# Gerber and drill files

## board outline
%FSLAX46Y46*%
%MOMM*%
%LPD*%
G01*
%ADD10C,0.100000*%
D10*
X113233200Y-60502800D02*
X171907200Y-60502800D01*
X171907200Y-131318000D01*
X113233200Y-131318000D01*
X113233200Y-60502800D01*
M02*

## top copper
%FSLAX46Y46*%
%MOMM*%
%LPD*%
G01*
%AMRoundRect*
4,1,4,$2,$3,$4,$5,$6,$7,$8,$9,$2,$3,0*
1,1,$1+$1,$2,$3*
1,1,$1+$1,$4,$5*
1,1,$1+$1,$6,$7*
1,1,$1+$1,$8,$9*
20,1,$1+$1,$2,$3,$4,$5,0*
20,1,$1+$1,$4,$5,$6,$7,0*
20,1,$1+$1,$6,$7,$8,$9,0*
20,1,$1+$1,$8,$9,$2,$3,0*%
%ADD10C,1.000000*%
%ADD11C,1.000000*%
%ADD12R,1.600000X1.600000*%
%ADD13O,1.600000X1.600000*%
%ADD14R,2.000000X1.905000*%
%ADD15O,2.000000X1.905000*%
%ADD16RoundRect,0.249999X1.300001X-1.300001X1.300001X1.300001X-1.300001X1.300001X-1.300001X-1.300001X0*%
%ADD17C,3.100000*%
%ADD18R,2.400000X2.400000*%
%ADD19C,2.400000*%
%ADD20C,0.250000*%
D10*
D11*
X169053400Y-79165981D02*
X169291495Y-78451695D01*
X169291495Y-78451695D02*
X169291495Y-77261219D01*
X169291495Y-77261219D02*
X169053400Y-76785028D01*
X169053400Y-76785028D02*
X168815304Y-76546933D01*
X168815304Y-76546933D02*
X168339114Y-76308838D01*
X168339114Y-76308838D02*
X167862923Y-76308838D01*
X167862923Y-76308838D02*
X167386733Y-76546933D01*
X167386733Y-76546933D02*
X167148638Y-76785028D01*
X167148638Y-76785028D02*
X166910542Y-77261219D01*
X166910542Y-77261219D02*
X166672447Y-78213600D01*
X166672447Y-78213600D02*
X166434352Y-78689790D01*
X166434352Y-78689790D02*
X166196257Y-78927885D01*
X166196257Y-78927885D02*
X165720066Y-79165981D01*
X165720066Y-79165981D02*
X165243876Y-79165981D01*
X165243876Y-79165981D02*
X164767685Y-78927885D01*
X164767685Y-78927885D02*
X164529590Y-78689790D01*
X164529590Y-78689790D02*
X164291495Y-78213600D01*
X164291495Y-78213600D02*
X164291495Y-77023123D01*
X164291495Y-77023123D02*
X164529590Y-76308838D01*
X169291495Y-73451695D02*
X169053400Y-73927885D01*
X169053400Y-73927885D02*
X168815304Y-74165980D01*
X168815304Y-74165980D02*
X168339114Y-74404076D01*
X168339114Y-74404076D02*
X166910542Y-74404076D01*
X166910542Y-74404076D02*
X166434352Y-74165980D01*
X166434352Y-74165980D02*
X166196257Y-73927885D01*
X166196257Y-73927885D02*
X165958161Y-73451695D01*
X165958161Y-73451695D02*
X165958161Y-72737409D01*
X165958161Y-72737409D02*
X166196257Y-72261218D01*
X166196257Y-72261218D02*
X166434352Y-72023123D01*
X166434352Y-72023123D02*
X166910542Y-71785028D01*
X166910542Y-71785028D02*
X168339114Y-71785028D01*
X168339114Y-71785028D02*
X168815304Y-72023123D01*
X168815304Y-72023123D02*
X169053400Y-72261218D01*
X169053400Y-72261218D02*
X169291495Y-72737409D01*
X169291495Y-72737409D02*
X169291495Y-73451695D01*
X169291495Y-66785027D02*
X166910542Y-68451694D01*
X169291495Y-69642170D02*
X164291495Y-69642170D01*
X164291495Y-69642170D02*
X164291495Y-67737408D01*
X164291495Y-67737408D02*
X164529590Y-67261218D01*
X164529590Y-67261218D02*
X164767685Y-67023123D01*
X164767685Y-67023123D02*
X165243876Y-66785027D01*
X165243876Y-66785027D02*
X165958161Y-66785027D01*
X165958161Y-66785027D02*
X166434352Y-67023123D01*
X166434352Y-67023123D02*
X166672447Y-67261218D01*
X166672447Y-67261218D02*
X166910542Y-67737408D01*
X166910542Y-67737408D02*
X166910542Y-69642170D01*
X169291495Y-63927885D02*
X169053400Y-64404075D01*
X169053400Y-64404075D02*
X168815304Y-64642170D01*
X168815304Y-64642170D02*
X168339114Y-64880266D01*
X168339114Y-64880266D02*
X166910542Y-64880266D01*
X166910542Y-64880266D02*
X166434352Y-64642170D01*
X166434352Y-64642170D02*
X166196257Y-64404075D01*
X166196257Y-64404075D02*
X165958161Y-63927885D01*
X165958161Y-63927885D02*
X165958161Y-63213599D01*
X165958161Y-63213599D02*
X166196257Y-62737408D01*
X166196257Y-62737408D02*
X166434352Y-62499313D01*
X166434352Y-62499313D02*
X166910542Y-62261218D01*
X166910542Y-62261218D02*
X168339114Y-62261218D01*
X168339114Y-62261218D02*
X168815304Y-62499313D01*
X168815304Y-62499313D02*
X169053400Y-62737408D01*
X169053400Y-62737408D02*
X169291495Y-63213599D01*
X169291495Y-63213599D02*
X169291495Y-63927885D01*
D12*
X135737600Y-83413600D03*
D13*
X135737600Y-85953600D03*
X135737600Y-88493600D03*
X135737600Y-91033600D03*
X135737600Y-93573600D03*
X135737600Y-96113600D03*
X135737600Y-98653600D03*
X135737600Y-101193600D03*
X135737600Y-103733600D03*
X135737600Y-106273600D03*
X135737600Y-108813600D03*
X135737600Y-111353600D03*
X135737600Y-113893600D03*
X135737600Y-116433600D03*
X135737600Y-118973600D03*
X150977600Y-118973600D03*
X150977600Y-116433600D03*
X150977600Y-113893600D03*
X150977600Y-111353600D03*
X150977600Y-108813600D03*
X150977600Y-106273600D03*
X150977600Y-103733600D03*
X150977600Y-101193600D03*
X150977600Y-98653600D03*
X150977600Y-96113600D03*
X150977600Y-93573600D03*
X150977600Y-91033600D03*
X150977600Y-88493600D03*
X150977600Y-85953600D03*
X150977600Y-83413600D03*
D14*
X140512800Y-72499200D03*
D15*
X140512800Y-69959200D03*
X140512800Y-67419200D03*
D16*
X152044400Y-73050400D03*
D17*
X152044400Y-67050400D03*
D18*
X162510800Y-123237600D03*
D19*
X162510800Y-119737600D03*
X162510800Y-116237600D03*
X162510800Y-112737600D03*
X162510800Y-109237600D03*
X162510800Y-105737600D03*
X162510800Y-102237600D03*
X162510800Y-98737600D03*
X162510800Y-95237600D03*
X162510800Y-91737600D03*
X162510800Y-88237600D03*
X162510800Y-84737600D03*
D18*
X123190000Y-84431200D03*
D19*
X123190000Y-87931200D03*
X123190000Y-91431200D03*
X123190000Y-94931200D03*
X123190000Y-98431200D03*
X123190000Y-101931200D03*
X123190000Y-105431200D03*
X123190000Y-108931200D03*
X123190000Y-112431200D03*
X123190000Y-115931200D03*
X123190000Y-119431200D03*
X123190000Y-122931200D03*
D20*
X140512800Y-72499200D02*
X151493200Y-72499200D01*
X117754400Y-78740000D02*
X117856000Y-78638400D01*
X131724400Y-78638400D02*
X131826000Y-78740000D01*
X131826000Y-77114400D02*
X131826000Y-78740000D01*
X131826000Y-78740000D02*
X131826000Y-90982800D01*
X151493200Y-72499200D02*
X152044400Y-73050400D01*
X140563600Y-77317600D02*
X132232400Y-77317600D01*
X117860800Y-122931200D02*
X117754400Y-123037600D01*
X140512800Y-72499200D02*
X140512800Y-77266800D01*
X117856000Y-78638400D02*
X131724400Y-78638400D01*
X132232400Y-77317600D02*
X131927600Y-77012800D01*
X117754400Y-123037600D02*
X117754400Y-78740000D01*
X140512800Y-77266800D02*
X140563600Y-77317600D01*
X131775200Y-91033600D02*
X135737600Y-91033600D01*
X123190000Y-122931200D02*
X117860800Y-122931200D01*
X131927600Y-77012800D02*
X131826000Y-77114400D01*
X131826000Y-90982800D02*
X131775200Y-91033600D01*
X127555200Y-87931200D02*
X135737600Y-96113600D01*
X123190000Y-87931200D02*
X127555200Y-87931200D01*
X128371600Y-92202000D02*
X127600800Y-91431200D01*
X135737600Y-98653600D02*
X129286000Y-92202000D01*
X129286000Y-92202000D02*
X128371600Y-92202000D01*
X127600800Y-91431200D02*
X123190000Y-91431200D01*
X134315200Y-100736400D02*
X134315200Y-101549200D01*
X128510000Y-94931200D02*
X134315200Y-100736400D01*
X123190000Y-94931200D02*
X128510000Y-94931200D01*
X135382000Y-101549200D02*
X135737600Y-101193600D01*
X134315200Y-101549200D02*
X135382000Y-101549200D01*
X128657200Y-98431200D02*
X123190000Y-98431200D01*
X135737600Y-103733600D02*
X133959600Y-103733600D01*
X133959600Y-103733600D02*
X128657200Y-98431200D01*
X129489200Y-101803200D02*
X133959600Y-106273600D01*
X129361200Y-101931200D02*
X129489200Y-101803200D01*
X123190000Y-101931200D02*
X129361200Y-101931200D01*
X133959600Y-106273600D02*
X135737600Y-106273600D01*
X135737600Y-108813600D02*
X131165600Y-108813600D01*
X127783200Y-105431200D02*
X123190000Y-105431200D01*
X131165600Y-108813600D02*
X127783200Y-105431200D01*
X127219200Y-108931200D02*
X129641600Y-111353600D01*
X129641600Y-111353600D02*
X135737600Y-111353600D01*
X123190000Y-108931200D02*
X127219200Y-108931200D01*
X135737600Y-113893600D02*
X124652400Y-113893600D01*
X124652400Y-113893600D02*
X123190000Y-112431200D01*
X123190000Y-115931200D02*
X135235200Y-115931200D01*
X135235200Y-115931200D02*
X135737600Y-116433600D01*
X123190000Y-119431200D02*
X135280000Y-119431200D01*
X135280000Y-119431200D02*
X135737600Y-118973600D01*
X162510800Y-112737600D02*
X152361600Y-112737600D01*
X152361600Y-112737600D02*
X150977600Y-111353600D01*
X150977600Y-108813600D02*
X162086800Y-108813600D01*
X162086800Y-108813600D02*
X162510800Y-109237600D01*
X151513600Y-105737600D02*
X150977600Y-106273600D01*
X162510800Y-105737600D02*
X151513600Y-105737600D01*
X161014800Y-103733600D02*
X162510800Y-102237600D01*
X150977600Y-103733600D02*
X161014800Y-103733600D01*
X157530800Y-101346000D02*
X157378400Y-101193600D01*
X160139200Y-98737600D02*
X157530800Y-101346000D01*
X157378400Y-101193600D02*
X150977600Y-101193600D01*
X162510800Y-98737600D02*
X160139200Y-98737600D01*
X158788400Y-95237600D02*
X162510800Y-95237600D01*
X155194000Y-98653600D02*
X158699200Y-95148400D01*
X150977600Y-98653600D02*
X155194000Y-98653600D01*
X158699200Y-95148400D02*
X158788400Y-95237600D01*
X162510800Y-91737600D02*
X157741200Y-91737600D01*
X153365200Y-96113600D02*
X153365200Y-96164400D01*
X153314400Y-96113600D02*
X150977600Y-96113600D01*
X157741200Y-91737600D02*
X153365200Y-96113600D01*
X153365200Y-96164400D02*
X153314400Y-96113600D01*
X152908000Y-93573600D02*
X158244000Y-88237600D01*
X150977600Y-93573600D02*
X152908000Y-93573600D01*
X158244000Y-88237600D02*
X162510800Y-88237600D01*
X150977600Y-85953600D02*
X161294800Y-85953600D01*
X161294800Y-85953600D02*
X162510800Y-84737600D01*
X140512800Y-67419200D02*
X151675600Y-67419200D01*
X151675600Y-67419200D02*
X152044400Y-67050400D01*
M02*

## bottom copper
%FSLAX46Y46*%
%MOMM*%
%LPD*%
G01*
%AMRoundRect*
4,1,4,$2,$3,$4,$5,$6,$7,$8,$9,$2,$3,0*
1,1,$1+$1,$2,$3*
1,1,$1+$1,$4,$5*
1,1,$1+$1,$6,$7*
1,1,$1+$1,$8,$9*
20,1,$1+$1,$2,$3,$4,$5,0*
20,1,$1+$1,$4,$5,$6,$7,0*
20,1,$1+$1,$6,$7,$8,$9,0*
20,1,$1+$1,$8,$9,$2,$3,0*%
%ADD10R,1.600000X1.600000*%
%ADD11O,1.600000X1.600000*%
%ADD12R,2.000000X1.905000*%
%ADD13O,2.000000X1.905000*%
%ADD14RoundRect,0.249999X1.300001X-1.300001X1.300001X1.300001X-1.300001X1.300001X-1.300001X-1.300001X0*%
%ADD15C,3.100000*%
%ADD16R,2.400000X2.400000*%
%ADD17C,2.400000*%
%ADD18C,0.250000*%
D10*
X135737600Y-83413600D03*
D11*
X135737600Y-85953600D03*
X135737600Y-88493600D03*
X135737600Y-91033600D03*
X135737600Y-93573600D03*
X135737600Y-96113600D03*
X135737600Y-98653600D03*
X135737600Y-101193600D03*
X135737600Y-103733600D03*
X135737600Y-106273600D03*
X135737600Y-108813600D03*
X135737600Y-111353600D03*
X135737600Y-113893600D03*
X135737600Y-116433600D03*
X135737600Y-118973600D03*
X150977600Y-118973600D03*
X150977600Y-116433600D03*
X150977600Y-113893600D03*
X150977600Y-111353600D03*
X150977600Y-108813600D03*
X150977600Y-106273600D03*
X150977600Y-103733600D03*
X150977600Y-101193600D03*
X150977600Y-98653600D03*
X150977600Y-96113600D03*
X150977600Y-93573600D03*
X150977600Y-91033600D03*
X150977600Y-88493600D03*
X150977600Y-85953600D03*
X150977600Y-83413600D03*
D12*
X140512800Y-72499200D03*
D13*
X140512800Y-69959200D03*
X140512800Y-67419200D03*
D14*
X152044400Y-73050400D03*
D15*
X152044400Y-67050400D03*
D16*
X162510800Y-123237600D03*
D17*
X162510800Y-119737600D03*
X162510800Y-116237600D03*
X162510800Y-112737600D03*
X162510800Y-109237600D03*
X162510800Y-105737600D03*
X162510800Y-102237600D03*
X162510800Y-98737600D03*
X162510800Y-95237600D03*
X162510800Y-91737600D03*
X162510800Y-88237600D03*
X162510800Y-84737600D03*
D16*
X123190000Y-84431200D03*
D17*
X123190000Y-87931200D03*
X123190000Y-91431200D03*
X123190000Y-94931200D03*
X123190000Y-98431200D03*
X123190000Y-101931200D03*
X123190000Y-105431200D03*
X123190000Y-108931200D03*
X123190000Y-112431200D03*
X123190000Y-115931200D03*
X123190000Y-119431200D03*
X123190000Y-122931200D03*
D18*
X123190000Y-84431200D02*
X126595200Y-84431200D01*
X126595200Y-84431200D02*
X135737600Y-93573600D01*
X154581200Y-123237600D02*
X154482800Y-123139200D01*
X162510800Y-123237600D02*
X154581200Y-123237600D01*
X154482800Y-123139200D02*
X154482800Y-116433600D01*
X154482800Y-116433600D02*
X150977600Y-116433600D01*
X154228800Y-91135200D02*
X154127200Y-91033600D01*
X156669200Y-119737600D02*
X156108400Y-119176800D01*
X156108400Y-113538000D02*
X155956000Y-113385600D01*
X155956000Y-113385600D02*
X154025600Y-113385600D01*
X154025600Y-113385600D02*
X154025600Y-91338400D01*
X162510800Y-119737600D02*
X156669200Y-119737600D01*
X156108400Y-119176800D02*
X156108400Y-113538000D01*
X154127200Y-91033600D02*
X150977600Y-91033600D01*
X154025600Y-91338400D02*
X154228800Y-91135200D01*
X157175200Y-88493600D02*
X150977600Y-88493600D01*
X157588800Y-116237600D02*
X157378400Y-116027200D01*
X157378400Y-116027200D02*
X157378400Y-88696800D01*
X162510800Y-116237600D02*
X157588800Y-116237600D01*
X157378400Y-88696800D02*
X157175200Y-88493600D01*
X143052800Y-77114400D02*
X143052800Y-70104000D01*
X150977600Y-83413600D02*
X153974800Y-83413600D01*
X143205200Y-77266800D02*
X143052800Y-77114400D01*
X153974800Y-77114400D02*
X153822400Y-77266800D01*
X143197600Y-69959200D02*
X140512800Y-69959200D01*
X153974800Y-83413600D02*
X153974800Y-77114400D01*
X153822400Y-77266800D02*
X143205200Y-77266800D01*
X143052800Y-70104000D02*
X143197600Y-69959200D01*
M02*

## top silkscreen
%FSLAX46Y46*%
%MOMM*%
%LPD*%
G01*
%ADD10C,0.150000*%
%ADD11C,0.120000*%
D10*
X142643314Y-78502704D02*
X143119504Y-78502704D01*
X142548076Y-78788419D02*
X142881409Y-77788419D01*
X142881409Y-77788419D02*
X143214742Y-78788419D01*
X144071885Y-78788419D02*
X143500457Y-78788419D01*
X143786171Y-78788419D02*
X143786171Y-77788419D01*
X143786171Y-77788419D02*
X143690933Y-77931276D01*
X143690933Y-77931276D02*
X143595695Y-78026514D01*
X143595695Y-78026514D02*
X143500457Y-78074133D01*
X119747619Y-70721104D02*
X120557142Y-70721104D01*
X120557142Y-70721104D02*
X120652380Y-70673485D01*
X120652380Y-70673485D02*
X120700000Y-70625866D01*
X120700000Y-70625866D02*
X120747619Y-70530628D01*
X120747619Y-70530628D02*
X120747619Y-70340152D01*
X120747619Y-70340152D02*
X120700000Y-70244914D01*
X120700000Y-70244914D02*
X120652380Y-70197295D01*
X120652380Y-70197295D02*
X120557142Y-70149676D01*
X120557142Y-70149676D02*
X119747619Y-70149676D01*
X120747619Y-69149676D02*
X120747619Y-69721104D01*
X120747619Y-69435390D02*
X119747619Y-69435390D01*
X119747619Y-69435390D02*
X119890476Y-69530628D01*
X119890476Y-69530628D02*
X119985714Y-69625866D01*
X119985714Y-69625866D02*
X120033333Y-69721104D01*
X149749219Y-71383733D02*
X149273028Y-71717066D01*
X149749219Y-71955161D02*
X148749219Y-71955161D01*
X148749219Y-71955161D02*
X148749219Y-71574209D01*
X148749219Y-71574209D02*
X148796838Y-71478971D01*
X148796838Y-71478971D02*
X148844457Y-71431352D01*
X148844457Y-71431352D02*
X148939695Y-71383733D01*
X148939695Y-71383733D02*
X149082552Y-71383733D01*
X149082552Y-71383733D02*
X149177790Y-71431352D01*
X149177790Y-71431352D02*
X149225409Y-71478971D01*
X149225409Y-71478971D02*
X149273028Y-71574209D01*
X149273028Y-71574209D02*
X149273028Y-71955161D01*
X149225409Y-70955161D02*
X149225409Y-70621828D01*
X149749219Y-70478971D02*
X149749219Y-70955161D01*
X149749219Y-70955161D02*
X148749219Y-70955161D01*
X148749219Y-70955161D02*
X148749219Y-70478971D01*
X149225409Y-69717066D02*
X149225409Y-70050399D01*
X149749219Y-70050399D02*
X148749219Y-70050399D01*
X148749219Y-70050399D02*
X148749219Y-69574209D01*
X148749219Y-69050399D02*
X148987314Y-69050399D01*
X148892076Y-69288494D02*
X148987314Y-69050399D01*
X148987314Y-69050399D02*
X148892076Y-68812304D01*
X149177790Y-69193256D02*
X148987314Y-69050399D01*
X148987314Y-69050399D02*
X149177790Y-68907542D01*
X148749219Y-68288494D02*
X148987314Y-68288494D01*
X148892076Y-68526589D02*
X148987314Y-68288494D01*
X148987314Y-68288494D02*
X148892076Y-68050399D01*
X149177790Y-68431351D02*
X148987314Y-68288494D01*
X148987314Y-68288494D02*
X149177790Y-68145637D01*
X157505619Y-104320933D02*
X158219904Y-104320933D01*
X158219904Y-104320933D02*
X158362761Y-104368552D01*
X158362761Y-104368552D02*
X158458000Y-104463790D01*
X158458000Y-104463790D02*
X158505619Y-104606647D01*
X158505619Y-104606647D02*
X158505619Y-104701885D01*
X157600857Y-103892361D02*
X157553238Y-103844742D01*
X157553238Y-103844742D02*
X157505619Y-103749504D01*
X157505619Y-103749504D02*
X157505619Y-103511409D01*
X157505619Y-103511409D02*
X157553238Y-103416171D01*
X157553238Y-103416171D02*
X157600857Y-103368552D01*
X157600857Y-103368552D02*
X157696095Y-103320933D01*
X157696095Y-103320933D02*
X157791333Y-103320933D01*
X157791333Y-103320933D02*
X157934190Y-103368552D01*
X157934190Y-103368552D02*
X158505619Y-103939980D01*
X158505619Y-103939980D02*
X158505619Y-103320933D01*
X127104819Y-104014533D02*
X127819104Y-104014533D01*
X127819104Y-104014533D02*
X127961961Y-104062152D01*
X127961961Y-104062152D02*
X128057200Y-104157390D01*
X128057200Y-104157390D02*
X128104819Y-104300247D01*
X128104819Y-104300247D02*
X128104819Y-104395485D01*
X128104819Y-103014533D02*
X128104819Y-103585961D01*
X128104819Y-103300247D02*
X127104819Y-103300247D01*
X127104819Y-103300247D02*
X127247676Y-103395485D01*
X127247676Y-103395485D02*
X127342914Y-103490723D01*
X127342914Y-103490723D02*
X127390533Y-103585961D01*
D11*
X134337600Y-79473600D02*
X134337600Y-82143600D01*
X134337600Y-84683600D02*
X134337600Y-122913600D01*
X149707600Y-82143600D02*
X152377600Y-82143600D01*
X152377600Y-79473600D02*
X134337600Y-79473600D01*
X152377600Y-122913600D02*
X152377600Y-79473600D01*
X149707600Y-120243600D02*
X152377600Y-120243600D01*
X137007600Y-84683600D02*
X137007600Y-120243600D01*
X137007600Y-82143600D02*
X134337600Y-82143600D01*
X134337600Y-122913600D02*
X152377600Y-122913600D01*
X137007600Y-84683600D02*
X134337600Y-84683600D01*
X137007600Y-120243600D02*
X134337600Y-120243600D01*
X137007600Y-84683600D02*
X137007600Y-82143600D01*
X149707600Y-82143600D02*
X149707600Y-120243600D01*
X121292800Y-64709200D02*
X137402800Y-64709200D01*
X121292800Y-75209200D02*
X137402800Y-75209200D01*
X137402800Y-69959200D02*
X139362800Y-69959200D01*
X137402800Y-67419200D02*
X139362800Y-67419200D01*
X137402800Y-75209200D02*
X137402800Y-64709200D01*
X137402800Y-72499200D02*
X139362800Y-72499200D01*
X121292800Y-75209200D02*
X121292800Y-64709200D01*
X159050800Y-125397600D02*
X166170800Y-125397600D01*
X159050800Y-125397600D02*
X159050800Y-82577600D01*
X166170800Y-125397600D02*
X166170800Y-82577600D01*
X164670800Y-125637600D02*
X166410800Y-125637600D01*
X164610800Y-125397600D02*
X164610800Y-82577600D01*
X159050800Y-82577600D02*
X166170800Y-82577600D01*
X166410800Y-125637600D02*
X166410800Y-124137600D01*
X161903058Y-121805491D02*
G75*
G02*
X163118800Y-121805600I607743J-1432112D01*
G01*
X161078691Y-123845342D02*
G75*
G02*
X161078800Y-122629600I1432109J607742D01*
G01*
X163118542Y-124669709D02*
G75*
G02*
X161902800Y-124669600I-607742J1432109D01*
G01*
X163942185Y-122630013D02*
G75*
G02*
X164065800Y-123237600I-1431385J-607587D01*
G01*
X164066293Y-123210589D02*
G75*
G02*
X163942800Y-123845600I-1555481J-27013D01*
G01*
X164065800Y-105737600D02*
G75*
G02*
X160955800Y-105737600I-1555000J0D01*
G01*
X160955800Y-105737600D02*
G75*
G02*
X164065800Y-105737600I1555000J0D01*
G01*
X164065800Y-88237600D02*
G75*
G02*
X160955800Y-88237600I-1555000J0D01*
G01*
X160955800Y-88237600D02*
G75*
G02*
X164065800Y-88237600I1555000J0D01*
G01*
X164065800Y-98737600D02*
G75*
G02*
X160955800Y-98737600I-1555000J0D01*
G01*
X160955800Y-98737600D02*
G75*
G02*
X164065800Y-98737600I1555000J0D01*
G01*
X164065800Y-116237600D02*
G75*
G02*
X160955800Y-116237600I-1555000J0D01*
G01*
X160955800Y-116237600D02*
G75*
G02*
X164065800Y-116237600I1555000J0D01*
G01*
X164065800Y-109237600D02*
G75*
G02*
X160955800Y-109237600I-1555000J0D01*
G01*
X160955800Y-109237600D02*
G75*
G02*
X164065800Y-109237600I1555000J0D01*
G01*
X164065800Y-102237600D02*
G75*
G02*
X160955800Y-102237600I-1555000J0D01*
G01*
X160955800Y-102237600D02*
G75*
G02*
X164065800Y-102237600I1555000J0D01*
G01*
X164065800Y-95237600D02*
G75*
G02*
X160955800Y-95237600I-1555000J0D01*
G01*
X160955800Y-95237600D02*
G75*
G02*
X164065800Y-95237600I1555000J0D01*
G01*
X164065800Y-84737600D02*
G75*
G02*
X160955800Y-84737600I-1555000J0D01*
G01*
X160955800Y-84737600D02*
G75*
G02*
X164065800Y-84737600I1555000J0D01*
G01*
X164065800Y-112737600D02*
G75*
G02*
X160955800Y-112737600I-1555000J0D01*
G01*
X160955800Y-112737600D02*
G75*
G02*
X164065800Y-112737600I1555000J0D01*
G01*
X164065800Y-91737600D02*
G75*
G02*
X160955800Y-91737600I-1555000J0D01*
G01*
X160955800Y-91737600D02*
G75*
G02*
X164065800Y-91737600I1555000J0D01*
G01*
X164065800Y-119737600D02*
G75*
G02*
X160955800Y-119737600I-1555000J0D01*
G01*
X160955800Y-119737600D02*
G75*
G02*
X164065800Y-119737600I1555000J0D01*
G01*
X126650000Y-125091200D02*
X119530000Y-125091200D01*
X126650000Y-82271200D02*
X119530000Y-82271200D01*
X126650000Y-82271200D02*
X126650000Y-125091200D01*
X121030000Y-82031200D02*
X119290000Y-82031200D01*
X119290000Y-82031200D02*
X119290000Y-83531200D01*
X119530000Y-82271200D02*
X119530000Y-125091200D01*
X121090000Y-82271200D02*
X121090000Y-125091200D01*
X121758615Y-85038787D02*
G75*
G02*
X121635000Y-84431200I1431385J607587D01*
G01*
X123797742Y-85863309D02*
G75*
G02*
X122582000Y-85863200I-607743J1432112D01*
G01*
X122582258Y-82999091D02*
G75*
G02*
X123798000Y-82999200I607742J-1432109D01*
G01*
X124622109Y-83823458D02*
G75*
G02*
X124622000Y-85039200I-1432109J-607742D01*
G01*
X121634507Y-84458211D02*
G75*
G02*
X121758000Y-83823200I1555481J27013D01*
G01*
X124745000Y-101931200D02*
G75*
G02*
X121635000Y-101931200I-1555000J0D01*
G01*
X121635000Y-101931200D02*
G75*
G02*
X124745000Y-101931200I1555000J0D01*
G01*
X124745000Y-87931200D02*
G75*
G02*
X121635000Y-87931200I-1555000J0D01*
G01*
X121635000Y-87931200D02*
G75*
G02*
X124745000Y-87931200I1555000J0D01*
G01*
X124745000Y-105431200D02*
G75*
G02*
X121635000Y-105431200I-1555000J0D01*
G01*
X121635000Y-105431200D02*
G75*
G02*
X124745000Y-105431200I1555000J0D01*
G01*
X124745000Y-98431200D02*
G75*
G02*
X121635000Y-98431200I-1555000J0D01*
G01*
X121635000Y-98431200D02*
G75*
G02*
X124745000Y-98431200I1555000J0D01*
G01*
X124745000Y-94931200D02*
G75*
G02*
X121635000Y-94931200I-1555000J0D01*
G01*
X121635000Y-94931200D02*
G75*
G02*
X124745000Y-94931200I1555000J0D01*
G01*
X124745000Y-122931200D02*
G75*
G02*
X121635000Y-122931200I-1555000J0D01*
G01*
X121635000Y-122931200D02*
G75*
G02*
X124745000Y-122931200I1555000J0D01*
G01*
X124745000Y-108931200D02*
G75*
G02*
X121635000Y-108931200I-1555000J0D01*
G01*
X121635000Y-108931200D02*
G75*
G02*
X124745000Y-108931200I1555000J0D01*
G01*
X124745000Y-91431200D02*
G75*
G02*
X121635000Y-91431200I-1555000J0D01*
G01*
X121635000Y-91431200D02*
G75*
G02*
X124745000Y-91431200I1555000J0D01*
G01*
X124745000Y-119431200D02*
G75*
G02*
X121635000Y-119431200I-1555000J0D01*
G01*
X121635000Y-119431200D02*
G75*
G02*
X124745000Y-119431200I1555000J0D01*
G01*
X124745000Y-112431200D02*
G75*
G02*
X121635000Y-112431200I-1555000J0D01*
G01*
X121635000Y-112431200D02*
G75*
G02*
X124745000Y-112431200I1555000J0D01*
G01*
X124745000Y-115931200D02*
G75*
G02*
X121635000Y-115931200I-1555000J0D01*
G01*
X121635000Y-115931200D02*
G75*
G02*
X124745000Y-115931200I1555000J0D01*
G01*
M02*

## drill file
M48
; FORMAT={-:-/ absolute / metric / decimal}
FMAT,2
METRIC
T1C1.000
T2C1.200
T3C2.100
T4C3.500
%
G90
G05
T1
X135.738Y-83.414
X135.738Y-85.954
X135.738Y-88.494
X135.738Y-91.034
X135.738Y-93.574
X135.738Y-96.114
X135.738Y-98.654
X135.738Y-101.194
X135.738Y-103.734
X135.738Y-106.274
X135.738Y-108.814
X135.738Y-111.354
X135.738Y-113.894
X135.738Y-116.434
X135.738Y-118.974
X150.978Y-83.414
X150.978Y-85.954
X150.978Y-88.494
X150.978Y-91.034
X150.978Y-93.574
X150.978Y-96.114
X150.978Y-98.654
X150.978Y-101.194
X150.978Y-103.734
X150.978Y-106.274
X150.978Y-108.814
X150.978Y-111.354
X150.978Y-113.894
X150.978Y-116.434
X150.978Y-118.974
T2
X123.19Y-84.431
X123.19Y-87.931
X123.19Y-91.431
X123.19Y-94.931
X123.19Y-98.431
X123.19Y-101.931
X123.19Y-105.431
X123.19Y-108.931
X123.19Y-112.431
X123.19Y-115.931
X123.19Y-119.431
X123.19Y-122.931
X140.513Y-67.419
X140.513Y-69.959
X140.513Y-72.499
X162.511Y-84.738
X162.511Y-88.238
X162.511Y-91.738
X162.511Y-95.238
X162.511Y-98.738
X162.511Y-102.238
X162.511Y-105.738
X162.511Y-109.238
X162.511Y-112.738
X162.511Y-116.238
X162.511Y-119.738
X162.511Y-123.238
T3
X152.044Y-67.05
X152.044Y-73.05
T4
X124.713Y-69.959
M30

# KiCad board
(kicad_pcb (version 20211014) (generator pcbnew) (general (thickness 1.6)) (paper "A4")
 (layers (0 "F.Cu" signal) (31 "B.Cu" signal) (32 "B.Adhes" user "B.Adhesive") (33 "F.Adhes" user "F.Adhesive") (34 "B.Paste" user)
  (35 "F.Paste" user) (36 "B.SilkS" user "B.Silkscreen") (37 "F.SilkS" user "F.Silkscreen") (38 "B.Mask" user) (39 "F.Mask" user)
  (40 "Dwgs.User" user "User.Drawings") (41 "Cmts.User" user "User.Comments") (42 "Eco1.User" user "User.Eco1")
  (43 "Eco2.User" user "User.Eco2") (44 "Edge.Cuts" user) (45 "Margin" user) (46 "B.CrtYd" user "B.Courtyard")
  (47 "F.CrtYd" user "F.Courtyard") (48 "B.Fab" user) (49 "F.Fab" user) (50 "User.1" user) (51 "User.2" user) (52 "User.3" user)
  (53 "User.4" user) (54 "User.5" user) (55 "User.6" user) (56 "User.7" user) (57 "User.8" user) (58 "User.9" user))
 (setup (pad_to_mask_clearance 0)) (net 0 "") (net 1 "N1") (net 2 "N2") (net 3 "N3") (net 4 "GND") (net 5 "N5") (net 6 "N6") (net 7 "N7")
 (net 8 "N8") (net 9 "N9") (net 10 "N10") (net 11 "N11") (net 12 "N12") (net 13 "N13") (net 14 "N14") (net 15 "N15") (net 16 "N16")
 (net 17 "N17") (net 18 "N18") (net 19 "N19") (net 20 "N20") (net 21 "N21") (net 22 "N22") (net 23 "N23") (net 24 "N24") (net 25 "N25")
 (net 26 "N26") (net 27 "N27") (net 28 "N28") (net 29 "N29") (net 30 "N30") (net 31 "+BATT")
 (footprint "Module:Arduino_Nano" (layer "F.Cu") (at 135.7376 83.4136)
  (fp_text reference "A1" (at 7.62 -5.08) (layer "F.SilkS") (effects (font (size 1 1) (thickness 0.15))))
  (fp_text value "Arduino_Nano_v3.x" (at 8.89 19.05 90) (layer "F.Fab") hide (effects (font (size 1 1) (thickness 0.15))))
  (fp_line (start -1.4 -3.94) (end -1.4 -1.27) (layer "F.SilkS") (width 0.12))
  (fp_line (start -1.4 1.27) (end -1.4 39.5) (layer "F.SilkS") (width 0.12))
  (fp_line (start 13.97 -1.27) (end 16.64 -1.27) (layer "F.SilkS") (width 0.12))
  (fp_line (start 16.64 -3.94) (end -1.4 -3.94) (layer "F.SilkS") (width 0.12))
  (fp_line (start 16.64 39.5) (end 16.64 -3.94) (layer "F.SilkS") (width 0.12))
  (fp_line (start 13.97 36.83) (end 16.64 36.83) (layer "F.SilkS") (width 0.12))
  (fp_line (start 1.27 1.27) (end 1.27 36.83) (layer "F.SilkS") (width 0.12))
  (fp_line (start 1.27 -1.27) (end -1.4 -1.27) (layer "F.SilkS") (width 0.12))
  (fp_line (start -1.4 39.5) (end 16.64 39.5) (layer "F.SilkS") (width 0.12))
  (fp_line (start 1.27 1.27) (end -1.4 1.27) (layer "F.SilkS") (width 0.12))
  (fp_line (start 1.27 36.83) (end -1.4 36.83) (layer "F.SilkS") (width 0.12))
  (fp_line (start 1.27 1.27) (end 1.27 -1.27) (layer "F.SilkS") (width 0.12))
  (fp_line (start 13.97 -1.27) (end 13.97 36.83) (layer "F.SilkS") (width 0.12))
  (pad "1" thru_hole rect (at 0 0) (size 1.6 1.6) (drill 1) (layers *.Cu *.Mask) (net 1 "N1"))
  (pad "2" thru_hole oval (at 0 2.54) (size 1.6 1.6) (drill 1) (layers *.Cu *.Mask) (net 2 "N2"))
  (pad "3" thru_hole oval (at 0 5.08) (size 1.6 1.6) (drill 1) (layers *.Cu *.Mask) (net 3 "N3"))
  (pad "4" thru_hole oval (at 0 7.62) (size 1.6 1.6) (drill 1) (layers *.Cu *.Mask) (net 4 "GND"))
  (pad "5" thru_hole oval (at 0 10.16) (size 1.6 1.6) (drill 1) (layers *.Cu *.Mask) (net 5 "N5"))
  (pad "6" thru_hole oval (at 0 12.7) (size 1.6 1.6) (drill 1) (layers *.Cu *.Mask) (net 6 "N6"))
  (pad "7" thru_hole oval (at 0 15.24) (size 1.6 1.6) (drill 1) (layers *.Cu *.Mask) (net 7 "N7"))
  (pad "8" thru_hole oval (at 0 17.78) (size 1.6 1.6) (drill 1) (layers *.Cu *.Mask) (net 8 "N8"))
  (pad "9" thru_hole oval (at 0 20.32) (size 1.6 1.6) (drill 1) (layers *.Cu *.Mask) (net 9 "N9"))
  (pad "10" thru_hole oval (at 0 22.86) (size 1.6 1.6) (drill 1) (layers *.Cu *.Mask) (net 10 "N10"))
  (pad "11" thru_hole oval (at 0 25.4) (size 1.6 1.6) (drill 1) (layers *.Cu *.Mask) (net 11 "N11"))
  (pad "12" thru_hole oval (at 0 27.94) (size 1.6 1.6) (drill 1) (layers *.Cu *.Mask) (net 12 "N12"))
  (pad "13" thru_hole oval (at 0 30.48) (size 1.6 1.6) (drill 1) (layers *.Cu *.Mask) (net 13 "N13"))
  (pad "14" thru_hole oval (at 0 33.02) (size 1.6 1.6) (drill 1) (layers *.Cu *.Mask) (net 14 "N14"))
  (pad "15" thru_hole oval (at 0 35.56) (size 1.6 1.6) (drill 1) (layers *.Cu *.Mask) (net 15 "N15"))
  (pad "16" thru_hole oval (at 15.24 35.56) (size 1.6 1.6) (drill 1) (layers *.Cu *.Mask) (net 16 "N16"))
  (pad "17" thru_hole oval (at 15.24 33.02) (size 1.6 1.6) (drill 1) (layers *.Cu *.Mask) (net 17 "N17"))
  (pad "18" thru_hole oval (at 15.24 30.48) (size 1.6 1.6) (drill 1) (layers *.Cu *.Mask) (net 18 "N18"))
  (pad "19" thru_hole oval (at 15.24 27.94) (size 1.6 1.6) (drill 1) (layers *.Cu *.Mask) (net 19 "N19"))
  (pad "20" thru_hole oval (at 15.24 25.4) (size 1.6 1.6) (drill 1) (layers *.Cu *.Mask) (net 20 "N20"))
  (pad "21" thru_hole oval (at 15.24 22.86) (size 1.6 1.6) (drill 1) (layers *.Cu *.Mask) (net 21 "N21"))
  (pad "22" thru_hole oval (at 15.24 20.32) (size 1.6 1.6) (drill 1) (layers *.Cu *.Mask) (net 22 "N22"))
  (pad "23" thru_hole oval (at 15.24 17.78) (size 1.6 1.6) (drill 1) (layers *.Cu *.Mask) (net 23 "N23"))
  (pad "24" thru_hole oval (at 15.24 15.24) (size 1.6 1.6) (drill 1) (layers *.Cu *.Mask) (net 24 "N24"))
  (pad "25" thru_hole oval (at 15.24 12.7) (size 1.6 1.6) (drill 1) (layers *.Cu *.Mask) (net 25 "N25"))
  (pad "26" thru_hole oval (at 15.24 10.16) (size 1.6 1.6) (drill 1) (layers *.Cu *.Mask) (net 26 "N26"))
  (pad "27" thru_hole oval (at 15.24 7.62) (size 1.6 1.6) (drill 1) (layers *.Cu *.Mask) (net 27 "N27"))
  (pad "28" thru_hole oval (at 15.24 5.08) (size 1.6 1.6) (drill 1) (layers *.Cu *.Mask) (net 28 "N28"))
  (pad "29" thru_hole oval (at 15.24 2.54) (size 1.6 1.6) (drill 1) (layers *.Cu *.Mask) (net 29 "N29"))
  (pad "30" thru_hole oval (at 15.24 0) (size 1.6 1.6) (drill 1) (layers *.Cu *.Mask) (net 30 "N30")))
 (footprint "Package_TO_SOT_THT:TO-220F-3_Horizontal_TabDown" (layer "F.Cu") (at 140.5128 72.4992 90)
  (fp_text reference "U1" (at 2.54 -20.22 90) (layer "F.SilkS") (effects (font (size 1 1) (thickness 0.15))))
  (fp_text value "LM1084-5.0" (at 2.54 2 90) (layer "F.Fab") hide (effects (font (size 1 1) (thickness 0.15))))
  (fp_line (start 7.79 -19.22) (end 7.79 -3.11) (layer "F.SilkS") (width 0.12))
  (fp_line (start -2.71 -19.22) (end -2.71 -3.11) (layer "F.SilkS") (width 0.12))
  (fp_line (start 2.54 -3.11) (end 2.54 -1.15) (layer "F.SilkS") (width 0.12))
  (fp_line (start 5.08 -3.11) (end 5.08 -1.15) (layer "F.SilkS") (width 0.12))
  (fp_line (start -2.71 -3.11) (end 7.79 -3.11) (layer "F.SilkS") (width 0.12))
  (fp_line (start 0 -3.11) (end 0 -1.15) (layer "F.SilkS") (width 0.12))
  (fp_line (start -2.71 -19.22) (end 7.79 -19.22) (layer "F.SilkS") (width 0.12))
  (pad "" np_thru_hole oval (at 2.54 -15.8 90) (size 3.5 3.5) (drill 3.5) (layers *.Cu *.Mask))
  (pad "1" thru_hole rect (at 0 0 90) (size 1.905 2) (drill 1.2) (layers *.Cu *.Mask) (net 4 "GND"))
  (pad "2" thru_hole oval (at 2.54 0 90) (size 1.905 2) (drill 1.2) (layers *.Cu *.Mask) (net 30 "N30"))
  (pad "3" thru_hole oval (at 5.08 0 90) (size 1.905 2) (drill 1.2) (layers *.Cu *.Mask) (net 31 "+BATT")))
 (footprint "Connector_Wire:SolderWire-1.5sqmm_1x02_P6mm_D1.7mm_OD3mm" (layer "F.Cu") (at 152.0444 73.0504 90)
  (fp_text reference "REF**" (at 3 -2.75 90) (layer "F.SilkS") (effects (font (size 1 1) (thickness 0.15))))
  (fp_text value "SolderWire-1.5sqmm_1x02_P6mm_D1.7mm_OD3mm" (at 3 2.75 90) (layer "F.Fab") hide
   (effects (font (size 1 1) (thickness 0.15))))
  (pad "1" thru_hole roundrect (at 0 0 90) (size 3.1 3.1) (drill 2.1) (layers *.Cu *.Mask) (roundrect_rratio 0.08064483871) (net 4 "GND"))
  (pad "2" thru_hole circle (at 6 0 90) (size 3.1 3.1) (drill 2.1) (layers *.Cu *.Mask) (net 31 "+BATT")))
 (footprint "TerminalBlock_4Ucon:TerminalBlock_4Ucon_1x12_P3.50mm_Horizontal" (layer "F.Cu") (at 162.5108 123.2376 90)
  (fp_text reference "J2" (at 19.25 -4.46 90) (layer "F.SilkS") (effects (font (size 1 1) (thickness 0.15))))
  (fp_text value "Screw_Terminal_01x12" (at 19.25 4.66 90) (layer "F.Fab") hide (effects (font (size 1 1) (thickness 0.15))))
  (fp_line (start -2.16 -3.46) (end -2.16 3.66) (layer "F.SilkS") (width 0.12))
  (fp_line (start -2.16 -3.46) (end 40.66 -3.46) (layer "F.SilkS") (width 0.12))
  (fp_line (start -2.16 3.66) (end 40.66 3.66) (layer "F.SilkS") (width 0.12))
  (fp_line (start -2.4 2.16) (end -2.4 3.9) (layer "F.SilkS") (width 0.12))
  (fp_line (start -2.16 2.1) (end 40.66 2.1) (layer "F.SilkS") (width 0.12))
  (fp_line (start 40.66 -3.46) (end 40.66 3.66) (layer "F.SilkS") (width 0.12))
  (fp_line (start -2.4 3.9) (end -0.9 3.9) (layer "F.SilkS") (width 0.12))
  (fp_arc (start 1.432109 -0.607742) (mid 1.555727 0.00014) (end 1.432 0.608) (layer "F.SilkS") (width 0.12))
  (fp_arc (start -0.607742 -1.432109) (mid 0.00014 -1.555727) (end 0.608 -1.432) (layer "F.SilkS") (width 0.12))
  (fp_arc (start -1.432109 0.607742) (mid -1.555727 -0.00014) (end -1.432 -0.608) (layer "F.SilkS") (width 0.12))
  (fp_arc (start 0.607587 1.431385) (mid 0.310017 1.523783) (end 0 1.555) (layer "F.SilkS") (width 0.12))
  (fp_arc (start 0.027011 1.555493) (mid -0.296984 1.527118) (end -0.608 1.432) (layer "F.SilkS") (width 0.12))
  (fp_circle (center 17.5 0) (end 19.055 0) (layer "F.SilkS") (width 0.12) (fill none))
  (fp_circle (center 35 0) (end 36.555 0) (layer "F.SilkS") (width 0.12) (fill none))
  (fp_circle (center 24.5 0) (end 26.055 0) (layer "F.SilkS") (width 0.12) (fill none))
  (fp_circle (center 7 0) (end 8.555 0) (layer "F.SilkS") (width 0.12) (fill none))
  (fp_circle (center 14 0) (end 15.555 0) (layer "F.SilkS") (width 0.12) (fill none))
  (fp_circle (center 21 0) (end 22.555 0) (layer "F.SilkS") (width 0.12) (fill none))
  (fp_circle (center 28 0) (end 29.555 0) (layer "F.SilkS") (width 0.12) (fill none))
  (fp_circle (center 38.5 0) (end 40.055 0) (layer "F.SilkS") (width 0.12) (fill none))
  (fp_circle (center 10.5 0) (end 12.055 0) (layer "F.SilkS") (width 0.12) (fill none))
  (fp_circle (center 31.5 0) (end 33.055 0) (layer "F.SilkS") (width 0.12) (fill none))
  (fp_circle (center 3.5 0) (end 5.055 0) (layer "F.SilkS") (width 0.12) (fill none))
  (pad "1" thru_hole rect (at 0 0 90) (size 2.4 2.4) (drill 1.2) (layers *.Cu *.Mask) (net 17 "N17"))
  (pad "2" thru_hole circle (at 3.5 0 90) (size 2.4 2.4) (drill 1.2) (layers *.Cu *.Mask) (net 27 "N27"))
  (pad "3" thru_hole circle (at 7 0 90) (size 2.4 2.4) (drill 1.2) (layers *.Cu *.Mask) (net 28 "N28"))
  (pad "4" thru_hole circle (at 10.5 0 90) (size 2.4 2.4) (drill 1.2) (layers *.Cu *.Mask) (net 19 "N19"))
  (pad "5" thru_hole circle (at 14 0 90) (size 2.4 2.4) (drill 1.2) (layers *.Cu *.Mask) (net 20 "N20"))
  (pad "6" thru_hole circle (at 17.5 0 90) (size 2.4 2.4) (drill 1.2) (layers *.Cu *.Mask) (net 21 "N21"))
  (pad "7" thru_hole circle (at 21 0 90) (size 2.4 2.4) (drill 1.2) (layers *.Cu *.Mask) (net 22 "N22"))
  (pad "8" thru_hole circle (at 24.5 0 90) (size 2.4 2.4) (drill 1.2) (layers *.Cu *.Mask) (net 23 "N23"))
  (pad "9" thru_hole circle (at 28 0 90) (size 2.4 2.4) (drill 1.2) (layers *.Cu *.Mask) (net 24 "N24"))
  (pad "10" thru_hole circle (at 31.5 0 90) (size 2.4 2.4) (drill 1.2) (layers *.Cu *.Mask) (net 25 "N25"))
  (pad "11" thru_hole circle (at 35 0 90) (size 2.4 2.4) (drill 1.2) (layers *.Cu *.Mask) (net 26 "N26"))
  (pad "12" thru_hole circle (at 38.5 0 90) (size 2.4 2.4) (drill 1.2) (layers *.Cu *.Mask) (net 29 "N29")))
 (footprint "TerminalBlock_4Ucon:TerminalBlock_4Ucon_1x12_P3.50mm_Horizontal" (layer "F.Cu") (at 123.19 84.4312 -90)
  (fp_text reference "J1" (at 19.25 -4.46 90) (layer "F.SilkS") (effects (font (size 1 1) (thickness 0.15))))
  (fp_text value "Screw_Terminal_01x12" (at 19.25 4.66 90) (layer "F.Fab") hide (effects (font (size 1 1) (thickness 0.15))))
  (fp_line (start 40.66 -3.46) (end 40.66 3.66) (layer "F.SilkS") (width 0.12))
  (fp_line (start -2.16 -3.46) (end -2.16 3.66) (layer "F.SilkS") (width 0.12))
  (fp_line (start -2.16 -3.46) (end 40.66 -3.46) (layer "F.SilkS") (width 0.12))
  (fp_line (start -2.4 2.16) (end -2.4 3.9) (layer "F.SilkS") (width 0.12))
  (fp_line (start -2.4 3.9) (end -0.9 3.9) (layer "F.SilkS") (width 0.12))
  (fp_line (start -2.16 3.66) (end 40.66 3.66) (layer "F.SilkS") (width 0.12))
  (fp_line (start -2.16 2.1) (end 40.66 2.1) (layer "F.SilkS") (width 0.12))
  (fp_arc (start 0.607587 1.431385) (mid 0.310017 1.523783) (end 0 1.555) (layer "F.SilkS") (width 0.12))
  (fp_arc (start 1.432109 -0.607742) (mid 1.555727 0.00014) (end 1.432 0.608) (layer "F.SilkS") (width 0.12))
  (fp_arc (start -1.432109 0.607742) (mid -1.555727 -0.00014) (end -1.432 -0.608) (layer "F.SilkS") (width 0.12))
  (fp_arc (start -0.607742 -1.432109) (mid 0.00014 -1.555727) (end 0.608 -1.432) (layer "F.SilkS") (width 0.12))
  (fp_arc (start 0.027011 1.555493) (mid -0.296984 1.527118) (end -0.608 1.432) (layer "F.SilkS") (width 0.12))
  (fp_circle (center 17.5 0) (end 19.055 0) (layer "F.SilkS") (width 0.12) (fill none))
  (fp_circle (center 3.5 0) (end 5.055 0) (layer "F.SilkS") (width 0.12) (fill none))
  (fp_circle (center 21 0) (end 22.555 0) (layer "F.SilkS") (width 0.12) (fill none))
  (fp_circle (center 14 0) (end 15.555 0) (layer "F.SilkS") (width 0.12) (fill none))
  (fp_circle (center 10.5 0) (end 12.055 0) (layer "F.SilkS") (width 0.12) (fill none))
  (fp_circle (center 38.5 0) (end 40.055 0) (layer "F.SilkS") (width 0.12) (fill none))
  (fp_circle (center 24.5 0) (end 26.055 0) (layer "F.SilkS") (width 0.12) (fill none))
  (fp_circle (center 7 0) (end 8.555 0) (layer "F.SilkS") (width 0.12) (fill none))
  (fp_circle (center 35 0) (end 36.555 0) (layer "F.SilkS") (width 0.12) (fill none))
  (fp_circle (center 28 0) (end 29.555 0) (layer "F.SilkS") (width 0.12) (fill none))
  (fp_circle (center 31.5 0) (end 33.055 0) (layer "F.SilkS") (width 0.12) (fill none))
  (pad "1" thru_hole rect (at 0 0 270) (size 2.4 2.4) (drill 1.2) (layers *.Cu *.Mask) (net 5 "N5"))
  (pad "2" thru_hole circle (at 3.5 0 270) (size 2.4 2.4) (drill 1.2) (layers *.Cu *.Mask) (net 6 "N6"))
  (pad "3" thru_hole circle (at 7 0 270) (size 2.4 2.4) (drill 1.2) (layers *.Cu *.Mask) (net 7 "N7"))
  (pad "4" thru_hole circle (at 10.5 0 270) (size 2.4 2.4) (drill 1.2) (layers *.Cu *.Mask) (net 8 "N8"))
  (pad "5" thru_hole circle (at 14 0 270) (size 2.4 2.4) (drill 1.2) (layers *.Cu *.Mask) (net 9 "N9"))
  (pad "6" thru_hole circle (at 17.5 0 270) (size 2.4 2.4) (drill 1.2) (layers *.Cu *.Mask) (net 10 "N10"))
  (pad "7" thru_hole circle (at 21 0 270) (size 2.4 2.4) (drill 1.2) (layers *.Cu *.Mask) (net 11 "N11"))
  (pad "8" thru_hole circle (at 24.5 0 270) (size 2.4 2.4) (drill 1.2) (layers *.Cu *.Mask) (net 12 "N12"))
  (pad "9" thru_hole circle (at 28 0 270) (size 2.4 2.4) (drill 1.2) (layers *.Cu *.Mask) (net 13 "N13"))
  (pad "10" thru_hole circle (at 31.5 0 270) (size 2.4 2.4) (drill 1.2) (layers *.Cu *.Mask) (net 14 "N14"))
  (pad "11" thru_hole circle (at 35 0 270) (size 2.4 2.4) (drill 1.2) (layers *.Cu *.Mask) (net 15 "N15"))
  (pad "12" thru_hole circle (at 38.5 0 270) (size 2.4 2.4) (drill 1.2) (layers *.Cu *.Mask) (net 4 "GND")))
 (gr_rect (start 171.9072 131.318) (end 113.2332 60.5028) (layer "Edge.Cuts") (width 0.1) (fill none))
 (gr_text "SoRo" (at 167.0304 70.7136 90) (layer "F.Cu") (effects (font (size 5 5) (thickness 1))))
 (segment (start 140.5128 72.4992) (end 151.4932 72.4992) (width 0.25) (layer "F.Cu") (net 4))
 (segment (start 117.7544 78.74) (end 117.856 78.6384) (width 0.25) (layer "F.Cu") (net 4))
 (segment (start 131.7244 78.6384) (end 131.826 78.74) (width 0.25) (layer "F.Cu") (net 4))
 (segment (start 131.826 77.1144) (end 131.826 78.74) (width 0.25) (layer "F.Cu") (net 4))
 (segment (start 131.826 78.74) (end 131.826 90.9828) (width 0.25) (layer "F.Cu") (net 4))
 (segment (start 151.4932 72.4992) (end 152.0444 73.0504) (width 0.25) (layer "F.Cu") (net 4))
 (segment (start 140.5636 77.3176) (end 132.2324 77.3176) (width 0.25) (layer "F.Cu") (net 4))
 (segment (start 117.8608 122.9312) (end 117.7544 123.0376) (width 0.25) (layer "F.Cu") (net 4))
 (segment (start 140.5128 72.4992) (end 140.5128 77.2668) (width 0.25) (layer "F.Cu") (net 4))
 (segment (start 117.856 78.6384) (end 131.7244 78.6384) (width 0.25) (layer "F.Cu") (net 4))
 (segment (start 132.2324 77.3176) (end 131.9276 77.0128) (width 0.25) (layer "F.Cu") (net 4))
 (segment (start 117.7544 123.0376) (end 117.7544 78.74) (width 0.25) (layer "F.Cu") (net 4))
 (segment (start 140.5128 77.2668) (end 140.5636 77.3176) (width 0.25) (layer "F.Cu") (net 4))
 (segment (start 131.7752 91.0336) (end 135.7376 91.0336) (width 0.25) (layer "F.Cu") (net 4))
 (segment (start 123.19 122.9312) (end 117.8608 122.9312) (width 0.25) (layer "F.Cu") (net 4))
 (segment (start 131.9276 77.0128) (end 131.826 77.1144) (width 0.25) (layer "F.Cu") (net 4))
 (segment (start 131.826 90.9828) (end 131.7752 91.0336) (width 0.25) (layer "F.Cu") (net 4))
 (segment (start 123.19 84.4312) (end 126.5952 84.4312) (width 0.25) (layer "B.Cu") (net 5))
 (segment (start 126.5952 84.4312) (end 135.7376 93.5736) (width 0.25) (layer "B.Cu") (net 5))
 (segment (start 127.5552 87.9312) (end 135.7376 96.1136) (width 0.25) (layer "F.Cu") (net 6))
 (segment (start 123.19 87.9312) (end 127.5552 87.9312) (width 0.25) (layer "F.Cu") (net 6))
 (segment (start 128.3716 92.202) (end 127.6008 91.4312) (width 0.25) (layer "F.Cu") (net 7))
 (segment (start 135.7376 98.6536) (end 129.286 92.202) (width 0.25) (layer "F.Cu") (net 7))
 (segment (start 129.286 92.202) (end 128.3716 92.202) (width 0.25) (layer "F.Cu") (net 7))
 (segment (start 127.6008 91.4312) (end 123.19 91.4312) (width 0.25) (layer "F.Cu") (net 7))
 (segment (start 134.3152 100.7364) (end 134.3152 101.5492) (width 0.25) (layer "F.Cu") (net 8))
 (segment (start 128.51 94.9312) (end 134.3152 100.7364) (width 0.25) (layer "F.Cu") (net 8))
 (segment (start 123.19 94.9312) (end 128.51 94.9312) (width 0.25) (layer "F.Cu") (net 8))
 (segment (start 135.382 101.5492) (end 135.7376 101.1936) (width 0.25) (layer "F.Cu") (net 8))
 (segment (start 134.3152 101.5492) (end 135.382 101.5492) (width 0.25) (layer "F.Cu") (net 8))
 (segment (start 128.6572 98.4312) (end 123.19 98.4312) (width 0.25) (layer "F.Cu") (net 9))
 (segment (start 135.7376 103.7336) (end 133.9596 103.7336) (width 0.25) (layer "F.Cu") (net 9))
 (segment (start 133.9596 103.7336) (end 128.6572 98.4312) (width 0.25) (layer "F.Cu") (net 9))
 (segment (start 129.4892 101.8032) (end 133.9596 106.2736) (width 0.25) (layer "F.Cu") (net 10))
 (segment (start 129.3612 101.9312) (end 129.4892 101.8032) (width 0.25) (layer "F.Cu") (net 10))
 (segment (start 123.19 101.9312) (end 129.3612 101.9312) (width 0.25) (layer "F.Cu") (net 10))
 (segment (start 133.9596 106.2736) (end 135.7376 106.2736) (width 0.25) (layer "F.Cu") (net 10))
 (segment (start 135.7376 108.8136) (end 131.1656 108.8136) (width 0.25) (layer "F.Cu") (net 11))
 (segment (start 127.7832 105.4312) (end 123.19 105.4312) (width 0.25) (layer "F.Cu") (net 11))
 (segment (start 131.1656 108.8136) (end 127.7832 105.4312) (width 0.25) (layer "F.Cu") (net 11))
 (segment (start 127.2192 108.9312) (end 129.6416 111.3536) (width 0.25) (layer "F.Cu") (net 12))
 (segment (start 129.6416 111.3536) (end 135.7376 111.3536) (width 0.25) (layer "F.Cu") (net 12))
 (segment (start 123.19 108.9312) (end 127.2192 108.9312) (width 0.25) (layer "F.Cu") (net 12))
 (segment (start 135.7376 113.8936) (end 124.6524 113.8936) (width 0.25) (layer "F.Cu") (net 13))
 (segment (start 124.6524 113.8936) (end 123.19 112.4312) (width 0.25) (layer "F.Cu") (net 13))
 (segment (start 123.19 115.9312) (end 135.2352 115.9312) (width 0.25) (layer "F.Cu") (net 14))
 (segment (start 135.2352 115.9312) (end 135.7376 116.4336) (width 0.25) (layer "F.Cu") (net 14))
 (segment (start 123.19 119.4312) (end 135.28 119.4312) (width 0.25) (layer "F.Cu") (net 15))
 (segment (start 135.28 119.4312) (end 135.7376 118.9736) (width 0.25) (layer "F.Cu") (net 15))
 (segment (start 154.5812 123.2376) (end 154.4828 123.1392) (width 0.25) (layer "B.Cu") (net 17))
 (segment (start 162.5108 123.2376) (end 154.5812 123.2376) (width 0.25) (layer "B.Cu") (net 17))
 (segment (start 154.4828 123.1392) (end 154.4828 116.4336) (width 0.25) (layer "B.Cu") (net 17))
 (segment (start 154.4828 116.4336) (end 150.9776 116.4336) (width 0.25) (layer "B.Cu") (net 17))
 (segment (start 162.5108 112.7376) (end 152.3616 112.7376) (width 0.25) (layer "F.Cu") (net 19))
 (segment (start 152.3616 112.7376) (end 150.9776 111.3536) (width 0.25) (layer "F.Cu") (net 19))
 (segment (start 150.9776 108.8136) (end 162.0868 108.8136) (width 0.25) (layer "F.Cu") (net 20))
 (segment (start 162.0868 108.8136) (end 162.5108 109.2376) (width 0.25) (layer "F.Cu") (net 20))
 (segment (start 151.5136 105.7376) (end 150.9776 106.2736) (width 0.25) (layer "F.Cu") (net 21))
 (segment (start 162.5108 105.7376) (end 151.5136 105.7376) (width 0.25) (layer "F.Cu") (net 21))
 (segment (start 161.0148 103.7336) (end 162.5108 102.2376) (width 0.25) (layer "F.Cu") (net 22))
 (segment (start 150.9776 103.7336) (end 161.0148 103.7336) (width 0.25) (layer "F.Cu") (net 22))
 (segment (start 157.5308 101.346) (end 157.3784 101.1936) (width 0.25) (layer "F.Cu") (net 23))
 (segment (start 160.1392 98.7376) (end 157.5308 101.346) (width 0.25) (layer "F.Cu") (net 23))
 (segment (start 157.3784 101.1936) (end 150.9776 101.1936) (width 0.25) (layer "F.Cu") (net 23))
 (segment (start 162.5108 98.7376) (end 160.1392 98.7376) (width 0.25) (layer "F.Cu") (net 23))
 (segment (start 158.7884 95.2376) (end 162.5108 95.2376) (width 0.25) (layer "F.Cu") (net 24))
 (segment (start 155.194 98.6536) (end 158.6992 95.1484) (width 0.25) (layer "F.Cu") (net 24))
 (segment (start 150.9776 98.6536) (end 155.194 98.6536) (width 0.25) (layer "F.Cu") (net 24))
 (segment (start 158.6992 95.1484) (end 158.7884 95.2376) (width 0.25) (layer "F.Cu") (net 24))
 (segment (start 162.5108 91.7376) (end 157.7412 91.7376) (width 0.25) (layer "F.Cu") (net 25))
 (segment (start 153.3652 96.1136) (end 153.3652 96.1644) (width 0.25) (layer "F.Cu") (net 25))
 (segment (start 153.3144 96.1136) (end 150.9776 96.1136) (width 0.25) (layer "F.Cu") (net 25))
 (segment (start 157.7412 91.7376) (end 153.3652 96.1136) (width 0.25) (layer "F.Cu") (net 25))
 (segment (start 153.3652 96.1644) (end 153.3144 96.1136) (width 0.25) (layer "F.Cu") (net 25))
 (segment (start 152.908 93.5736) (end 158.244 88.2376) (width 0.25) (layer "F.Cu") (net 26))
 (segment (start 150.9776 93.5736) (end 152.908 93.5736) (width 0.25) (layer "F.Cu") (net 26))
 (segment (start 158.244 88.2376) (end 162.5108 88.2376) (width 0.25) (layer "F.Cu") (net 26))
 (segment (start 154.2288 91.1352) (end 154.1272 91.0336) (width 0.25) (layer "B.Cu") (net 27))
 (segment (start 156.6692 119.7376) (end 156.1084 119.1768) (width 0.25) (layer "B.Cu") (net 27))
 (segment (start 156.1084 113.538) (end 155.956 113.3856) (width 0.25) (layer "B.Cu") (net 27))
 (segment (start 155.956 113.3856) (end 154.0256 113.3856) (width 0.25) (layer "B.Cu") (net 27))
 (segment (start 154.0256 113.3856) (end 154.0256 91.3384) (width 0.25) (layer "B.Cu") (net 27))
 (segment (start 162.5108 119.7376) (end 156.6692 119.7376) (width 0.25) (layer "B.Cu") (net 27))
 (segment (start 156.1084 119.1768) (end 156.1084 113.538) (width 0.25) (layer "B.Cu") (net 27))
 (segment (start 154.1272 91.0336) (end 150.9776 91.0336) (width 0.25) (layer "B.Cu") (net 27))
 (segment (start 154.0256 91.3384) (end 154.2288 91.1352) (width 0.25) (layer "B.Cu") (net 27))
 (segment (start 157.1752 88.4936) (end 150.9776 88.4936) (width 0.25) (layer "B.Cu") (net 28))
 (segment (start 157.5888 116.2376) (end 157.3784 116.0272) (width 0.25) (layer "B.Cu") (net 28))
 (segment (start 157.3784 116.0272) (end 157.3784 88.6968) (width 0.25) (layer "B.Cu") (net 28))
 (segment (start 162.5108 116.2376) (end 157.5888 116.2376) (width 0.25) (layer "B.Cu") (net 28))
 (segment (start 157.3784 88.6968) (end 157.1752 88.4936) (width 0.25) (layer "B.Cu") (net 28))
 (segment (start 150.9776 85.9536) (end 161.2948 85.9536) (width 0.25) (layer "F.Cu") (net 29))
 (segment (start 161.2948 85.9536) (end 162.5108 84.7376) (width 0.25) (layer "F.Cu") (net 29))
 (segment (start 143.0528 77.1144) (end 143.0528 70.104) (width 0.25) (layer "B.Cu") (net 30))
 (segment (start 150.9776 83.4136) (end 153.9748 83.4136) (width 0.25) (layer "B.Cu") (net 30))
 (segment (start 143.2052 77.2668) (end 143.0528 77.1144) (width 0.25) (layer "B.Cu") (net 30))
 (segment (start 153.9748 77.1144) (end 153.8224 77.2668) (width 0.25) (layer "B.Cu") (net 30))
 (segment (start 143.1976 69.9592) (end 140.5128 69.9592) (width 0.25) (layer "B.Cu") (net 30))
 (segment (start 153.9748 83.4136) (end 153.9748 77.1144) (width 0.25) (layer "B.Cu") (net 30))
 (segment (start 153.8224 77.2668) (end 143.2052 77.2668) (width 0.25) (layer "B.Cu") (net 30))
 (segment (start 143.0528 70.104) (end 143.1976 69.9592) (width 0.25) (layer "B.Cu") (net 30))
 (segment (start 140.5128 67.4192) (end 151.6756 67.4192) (width 0.25) (layer "F.Cu") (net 31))
 (segment (start 151.6756 67.4192) (end 152.0444 67.0504) (width 0.25) (layer "F.Cu") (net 31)))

